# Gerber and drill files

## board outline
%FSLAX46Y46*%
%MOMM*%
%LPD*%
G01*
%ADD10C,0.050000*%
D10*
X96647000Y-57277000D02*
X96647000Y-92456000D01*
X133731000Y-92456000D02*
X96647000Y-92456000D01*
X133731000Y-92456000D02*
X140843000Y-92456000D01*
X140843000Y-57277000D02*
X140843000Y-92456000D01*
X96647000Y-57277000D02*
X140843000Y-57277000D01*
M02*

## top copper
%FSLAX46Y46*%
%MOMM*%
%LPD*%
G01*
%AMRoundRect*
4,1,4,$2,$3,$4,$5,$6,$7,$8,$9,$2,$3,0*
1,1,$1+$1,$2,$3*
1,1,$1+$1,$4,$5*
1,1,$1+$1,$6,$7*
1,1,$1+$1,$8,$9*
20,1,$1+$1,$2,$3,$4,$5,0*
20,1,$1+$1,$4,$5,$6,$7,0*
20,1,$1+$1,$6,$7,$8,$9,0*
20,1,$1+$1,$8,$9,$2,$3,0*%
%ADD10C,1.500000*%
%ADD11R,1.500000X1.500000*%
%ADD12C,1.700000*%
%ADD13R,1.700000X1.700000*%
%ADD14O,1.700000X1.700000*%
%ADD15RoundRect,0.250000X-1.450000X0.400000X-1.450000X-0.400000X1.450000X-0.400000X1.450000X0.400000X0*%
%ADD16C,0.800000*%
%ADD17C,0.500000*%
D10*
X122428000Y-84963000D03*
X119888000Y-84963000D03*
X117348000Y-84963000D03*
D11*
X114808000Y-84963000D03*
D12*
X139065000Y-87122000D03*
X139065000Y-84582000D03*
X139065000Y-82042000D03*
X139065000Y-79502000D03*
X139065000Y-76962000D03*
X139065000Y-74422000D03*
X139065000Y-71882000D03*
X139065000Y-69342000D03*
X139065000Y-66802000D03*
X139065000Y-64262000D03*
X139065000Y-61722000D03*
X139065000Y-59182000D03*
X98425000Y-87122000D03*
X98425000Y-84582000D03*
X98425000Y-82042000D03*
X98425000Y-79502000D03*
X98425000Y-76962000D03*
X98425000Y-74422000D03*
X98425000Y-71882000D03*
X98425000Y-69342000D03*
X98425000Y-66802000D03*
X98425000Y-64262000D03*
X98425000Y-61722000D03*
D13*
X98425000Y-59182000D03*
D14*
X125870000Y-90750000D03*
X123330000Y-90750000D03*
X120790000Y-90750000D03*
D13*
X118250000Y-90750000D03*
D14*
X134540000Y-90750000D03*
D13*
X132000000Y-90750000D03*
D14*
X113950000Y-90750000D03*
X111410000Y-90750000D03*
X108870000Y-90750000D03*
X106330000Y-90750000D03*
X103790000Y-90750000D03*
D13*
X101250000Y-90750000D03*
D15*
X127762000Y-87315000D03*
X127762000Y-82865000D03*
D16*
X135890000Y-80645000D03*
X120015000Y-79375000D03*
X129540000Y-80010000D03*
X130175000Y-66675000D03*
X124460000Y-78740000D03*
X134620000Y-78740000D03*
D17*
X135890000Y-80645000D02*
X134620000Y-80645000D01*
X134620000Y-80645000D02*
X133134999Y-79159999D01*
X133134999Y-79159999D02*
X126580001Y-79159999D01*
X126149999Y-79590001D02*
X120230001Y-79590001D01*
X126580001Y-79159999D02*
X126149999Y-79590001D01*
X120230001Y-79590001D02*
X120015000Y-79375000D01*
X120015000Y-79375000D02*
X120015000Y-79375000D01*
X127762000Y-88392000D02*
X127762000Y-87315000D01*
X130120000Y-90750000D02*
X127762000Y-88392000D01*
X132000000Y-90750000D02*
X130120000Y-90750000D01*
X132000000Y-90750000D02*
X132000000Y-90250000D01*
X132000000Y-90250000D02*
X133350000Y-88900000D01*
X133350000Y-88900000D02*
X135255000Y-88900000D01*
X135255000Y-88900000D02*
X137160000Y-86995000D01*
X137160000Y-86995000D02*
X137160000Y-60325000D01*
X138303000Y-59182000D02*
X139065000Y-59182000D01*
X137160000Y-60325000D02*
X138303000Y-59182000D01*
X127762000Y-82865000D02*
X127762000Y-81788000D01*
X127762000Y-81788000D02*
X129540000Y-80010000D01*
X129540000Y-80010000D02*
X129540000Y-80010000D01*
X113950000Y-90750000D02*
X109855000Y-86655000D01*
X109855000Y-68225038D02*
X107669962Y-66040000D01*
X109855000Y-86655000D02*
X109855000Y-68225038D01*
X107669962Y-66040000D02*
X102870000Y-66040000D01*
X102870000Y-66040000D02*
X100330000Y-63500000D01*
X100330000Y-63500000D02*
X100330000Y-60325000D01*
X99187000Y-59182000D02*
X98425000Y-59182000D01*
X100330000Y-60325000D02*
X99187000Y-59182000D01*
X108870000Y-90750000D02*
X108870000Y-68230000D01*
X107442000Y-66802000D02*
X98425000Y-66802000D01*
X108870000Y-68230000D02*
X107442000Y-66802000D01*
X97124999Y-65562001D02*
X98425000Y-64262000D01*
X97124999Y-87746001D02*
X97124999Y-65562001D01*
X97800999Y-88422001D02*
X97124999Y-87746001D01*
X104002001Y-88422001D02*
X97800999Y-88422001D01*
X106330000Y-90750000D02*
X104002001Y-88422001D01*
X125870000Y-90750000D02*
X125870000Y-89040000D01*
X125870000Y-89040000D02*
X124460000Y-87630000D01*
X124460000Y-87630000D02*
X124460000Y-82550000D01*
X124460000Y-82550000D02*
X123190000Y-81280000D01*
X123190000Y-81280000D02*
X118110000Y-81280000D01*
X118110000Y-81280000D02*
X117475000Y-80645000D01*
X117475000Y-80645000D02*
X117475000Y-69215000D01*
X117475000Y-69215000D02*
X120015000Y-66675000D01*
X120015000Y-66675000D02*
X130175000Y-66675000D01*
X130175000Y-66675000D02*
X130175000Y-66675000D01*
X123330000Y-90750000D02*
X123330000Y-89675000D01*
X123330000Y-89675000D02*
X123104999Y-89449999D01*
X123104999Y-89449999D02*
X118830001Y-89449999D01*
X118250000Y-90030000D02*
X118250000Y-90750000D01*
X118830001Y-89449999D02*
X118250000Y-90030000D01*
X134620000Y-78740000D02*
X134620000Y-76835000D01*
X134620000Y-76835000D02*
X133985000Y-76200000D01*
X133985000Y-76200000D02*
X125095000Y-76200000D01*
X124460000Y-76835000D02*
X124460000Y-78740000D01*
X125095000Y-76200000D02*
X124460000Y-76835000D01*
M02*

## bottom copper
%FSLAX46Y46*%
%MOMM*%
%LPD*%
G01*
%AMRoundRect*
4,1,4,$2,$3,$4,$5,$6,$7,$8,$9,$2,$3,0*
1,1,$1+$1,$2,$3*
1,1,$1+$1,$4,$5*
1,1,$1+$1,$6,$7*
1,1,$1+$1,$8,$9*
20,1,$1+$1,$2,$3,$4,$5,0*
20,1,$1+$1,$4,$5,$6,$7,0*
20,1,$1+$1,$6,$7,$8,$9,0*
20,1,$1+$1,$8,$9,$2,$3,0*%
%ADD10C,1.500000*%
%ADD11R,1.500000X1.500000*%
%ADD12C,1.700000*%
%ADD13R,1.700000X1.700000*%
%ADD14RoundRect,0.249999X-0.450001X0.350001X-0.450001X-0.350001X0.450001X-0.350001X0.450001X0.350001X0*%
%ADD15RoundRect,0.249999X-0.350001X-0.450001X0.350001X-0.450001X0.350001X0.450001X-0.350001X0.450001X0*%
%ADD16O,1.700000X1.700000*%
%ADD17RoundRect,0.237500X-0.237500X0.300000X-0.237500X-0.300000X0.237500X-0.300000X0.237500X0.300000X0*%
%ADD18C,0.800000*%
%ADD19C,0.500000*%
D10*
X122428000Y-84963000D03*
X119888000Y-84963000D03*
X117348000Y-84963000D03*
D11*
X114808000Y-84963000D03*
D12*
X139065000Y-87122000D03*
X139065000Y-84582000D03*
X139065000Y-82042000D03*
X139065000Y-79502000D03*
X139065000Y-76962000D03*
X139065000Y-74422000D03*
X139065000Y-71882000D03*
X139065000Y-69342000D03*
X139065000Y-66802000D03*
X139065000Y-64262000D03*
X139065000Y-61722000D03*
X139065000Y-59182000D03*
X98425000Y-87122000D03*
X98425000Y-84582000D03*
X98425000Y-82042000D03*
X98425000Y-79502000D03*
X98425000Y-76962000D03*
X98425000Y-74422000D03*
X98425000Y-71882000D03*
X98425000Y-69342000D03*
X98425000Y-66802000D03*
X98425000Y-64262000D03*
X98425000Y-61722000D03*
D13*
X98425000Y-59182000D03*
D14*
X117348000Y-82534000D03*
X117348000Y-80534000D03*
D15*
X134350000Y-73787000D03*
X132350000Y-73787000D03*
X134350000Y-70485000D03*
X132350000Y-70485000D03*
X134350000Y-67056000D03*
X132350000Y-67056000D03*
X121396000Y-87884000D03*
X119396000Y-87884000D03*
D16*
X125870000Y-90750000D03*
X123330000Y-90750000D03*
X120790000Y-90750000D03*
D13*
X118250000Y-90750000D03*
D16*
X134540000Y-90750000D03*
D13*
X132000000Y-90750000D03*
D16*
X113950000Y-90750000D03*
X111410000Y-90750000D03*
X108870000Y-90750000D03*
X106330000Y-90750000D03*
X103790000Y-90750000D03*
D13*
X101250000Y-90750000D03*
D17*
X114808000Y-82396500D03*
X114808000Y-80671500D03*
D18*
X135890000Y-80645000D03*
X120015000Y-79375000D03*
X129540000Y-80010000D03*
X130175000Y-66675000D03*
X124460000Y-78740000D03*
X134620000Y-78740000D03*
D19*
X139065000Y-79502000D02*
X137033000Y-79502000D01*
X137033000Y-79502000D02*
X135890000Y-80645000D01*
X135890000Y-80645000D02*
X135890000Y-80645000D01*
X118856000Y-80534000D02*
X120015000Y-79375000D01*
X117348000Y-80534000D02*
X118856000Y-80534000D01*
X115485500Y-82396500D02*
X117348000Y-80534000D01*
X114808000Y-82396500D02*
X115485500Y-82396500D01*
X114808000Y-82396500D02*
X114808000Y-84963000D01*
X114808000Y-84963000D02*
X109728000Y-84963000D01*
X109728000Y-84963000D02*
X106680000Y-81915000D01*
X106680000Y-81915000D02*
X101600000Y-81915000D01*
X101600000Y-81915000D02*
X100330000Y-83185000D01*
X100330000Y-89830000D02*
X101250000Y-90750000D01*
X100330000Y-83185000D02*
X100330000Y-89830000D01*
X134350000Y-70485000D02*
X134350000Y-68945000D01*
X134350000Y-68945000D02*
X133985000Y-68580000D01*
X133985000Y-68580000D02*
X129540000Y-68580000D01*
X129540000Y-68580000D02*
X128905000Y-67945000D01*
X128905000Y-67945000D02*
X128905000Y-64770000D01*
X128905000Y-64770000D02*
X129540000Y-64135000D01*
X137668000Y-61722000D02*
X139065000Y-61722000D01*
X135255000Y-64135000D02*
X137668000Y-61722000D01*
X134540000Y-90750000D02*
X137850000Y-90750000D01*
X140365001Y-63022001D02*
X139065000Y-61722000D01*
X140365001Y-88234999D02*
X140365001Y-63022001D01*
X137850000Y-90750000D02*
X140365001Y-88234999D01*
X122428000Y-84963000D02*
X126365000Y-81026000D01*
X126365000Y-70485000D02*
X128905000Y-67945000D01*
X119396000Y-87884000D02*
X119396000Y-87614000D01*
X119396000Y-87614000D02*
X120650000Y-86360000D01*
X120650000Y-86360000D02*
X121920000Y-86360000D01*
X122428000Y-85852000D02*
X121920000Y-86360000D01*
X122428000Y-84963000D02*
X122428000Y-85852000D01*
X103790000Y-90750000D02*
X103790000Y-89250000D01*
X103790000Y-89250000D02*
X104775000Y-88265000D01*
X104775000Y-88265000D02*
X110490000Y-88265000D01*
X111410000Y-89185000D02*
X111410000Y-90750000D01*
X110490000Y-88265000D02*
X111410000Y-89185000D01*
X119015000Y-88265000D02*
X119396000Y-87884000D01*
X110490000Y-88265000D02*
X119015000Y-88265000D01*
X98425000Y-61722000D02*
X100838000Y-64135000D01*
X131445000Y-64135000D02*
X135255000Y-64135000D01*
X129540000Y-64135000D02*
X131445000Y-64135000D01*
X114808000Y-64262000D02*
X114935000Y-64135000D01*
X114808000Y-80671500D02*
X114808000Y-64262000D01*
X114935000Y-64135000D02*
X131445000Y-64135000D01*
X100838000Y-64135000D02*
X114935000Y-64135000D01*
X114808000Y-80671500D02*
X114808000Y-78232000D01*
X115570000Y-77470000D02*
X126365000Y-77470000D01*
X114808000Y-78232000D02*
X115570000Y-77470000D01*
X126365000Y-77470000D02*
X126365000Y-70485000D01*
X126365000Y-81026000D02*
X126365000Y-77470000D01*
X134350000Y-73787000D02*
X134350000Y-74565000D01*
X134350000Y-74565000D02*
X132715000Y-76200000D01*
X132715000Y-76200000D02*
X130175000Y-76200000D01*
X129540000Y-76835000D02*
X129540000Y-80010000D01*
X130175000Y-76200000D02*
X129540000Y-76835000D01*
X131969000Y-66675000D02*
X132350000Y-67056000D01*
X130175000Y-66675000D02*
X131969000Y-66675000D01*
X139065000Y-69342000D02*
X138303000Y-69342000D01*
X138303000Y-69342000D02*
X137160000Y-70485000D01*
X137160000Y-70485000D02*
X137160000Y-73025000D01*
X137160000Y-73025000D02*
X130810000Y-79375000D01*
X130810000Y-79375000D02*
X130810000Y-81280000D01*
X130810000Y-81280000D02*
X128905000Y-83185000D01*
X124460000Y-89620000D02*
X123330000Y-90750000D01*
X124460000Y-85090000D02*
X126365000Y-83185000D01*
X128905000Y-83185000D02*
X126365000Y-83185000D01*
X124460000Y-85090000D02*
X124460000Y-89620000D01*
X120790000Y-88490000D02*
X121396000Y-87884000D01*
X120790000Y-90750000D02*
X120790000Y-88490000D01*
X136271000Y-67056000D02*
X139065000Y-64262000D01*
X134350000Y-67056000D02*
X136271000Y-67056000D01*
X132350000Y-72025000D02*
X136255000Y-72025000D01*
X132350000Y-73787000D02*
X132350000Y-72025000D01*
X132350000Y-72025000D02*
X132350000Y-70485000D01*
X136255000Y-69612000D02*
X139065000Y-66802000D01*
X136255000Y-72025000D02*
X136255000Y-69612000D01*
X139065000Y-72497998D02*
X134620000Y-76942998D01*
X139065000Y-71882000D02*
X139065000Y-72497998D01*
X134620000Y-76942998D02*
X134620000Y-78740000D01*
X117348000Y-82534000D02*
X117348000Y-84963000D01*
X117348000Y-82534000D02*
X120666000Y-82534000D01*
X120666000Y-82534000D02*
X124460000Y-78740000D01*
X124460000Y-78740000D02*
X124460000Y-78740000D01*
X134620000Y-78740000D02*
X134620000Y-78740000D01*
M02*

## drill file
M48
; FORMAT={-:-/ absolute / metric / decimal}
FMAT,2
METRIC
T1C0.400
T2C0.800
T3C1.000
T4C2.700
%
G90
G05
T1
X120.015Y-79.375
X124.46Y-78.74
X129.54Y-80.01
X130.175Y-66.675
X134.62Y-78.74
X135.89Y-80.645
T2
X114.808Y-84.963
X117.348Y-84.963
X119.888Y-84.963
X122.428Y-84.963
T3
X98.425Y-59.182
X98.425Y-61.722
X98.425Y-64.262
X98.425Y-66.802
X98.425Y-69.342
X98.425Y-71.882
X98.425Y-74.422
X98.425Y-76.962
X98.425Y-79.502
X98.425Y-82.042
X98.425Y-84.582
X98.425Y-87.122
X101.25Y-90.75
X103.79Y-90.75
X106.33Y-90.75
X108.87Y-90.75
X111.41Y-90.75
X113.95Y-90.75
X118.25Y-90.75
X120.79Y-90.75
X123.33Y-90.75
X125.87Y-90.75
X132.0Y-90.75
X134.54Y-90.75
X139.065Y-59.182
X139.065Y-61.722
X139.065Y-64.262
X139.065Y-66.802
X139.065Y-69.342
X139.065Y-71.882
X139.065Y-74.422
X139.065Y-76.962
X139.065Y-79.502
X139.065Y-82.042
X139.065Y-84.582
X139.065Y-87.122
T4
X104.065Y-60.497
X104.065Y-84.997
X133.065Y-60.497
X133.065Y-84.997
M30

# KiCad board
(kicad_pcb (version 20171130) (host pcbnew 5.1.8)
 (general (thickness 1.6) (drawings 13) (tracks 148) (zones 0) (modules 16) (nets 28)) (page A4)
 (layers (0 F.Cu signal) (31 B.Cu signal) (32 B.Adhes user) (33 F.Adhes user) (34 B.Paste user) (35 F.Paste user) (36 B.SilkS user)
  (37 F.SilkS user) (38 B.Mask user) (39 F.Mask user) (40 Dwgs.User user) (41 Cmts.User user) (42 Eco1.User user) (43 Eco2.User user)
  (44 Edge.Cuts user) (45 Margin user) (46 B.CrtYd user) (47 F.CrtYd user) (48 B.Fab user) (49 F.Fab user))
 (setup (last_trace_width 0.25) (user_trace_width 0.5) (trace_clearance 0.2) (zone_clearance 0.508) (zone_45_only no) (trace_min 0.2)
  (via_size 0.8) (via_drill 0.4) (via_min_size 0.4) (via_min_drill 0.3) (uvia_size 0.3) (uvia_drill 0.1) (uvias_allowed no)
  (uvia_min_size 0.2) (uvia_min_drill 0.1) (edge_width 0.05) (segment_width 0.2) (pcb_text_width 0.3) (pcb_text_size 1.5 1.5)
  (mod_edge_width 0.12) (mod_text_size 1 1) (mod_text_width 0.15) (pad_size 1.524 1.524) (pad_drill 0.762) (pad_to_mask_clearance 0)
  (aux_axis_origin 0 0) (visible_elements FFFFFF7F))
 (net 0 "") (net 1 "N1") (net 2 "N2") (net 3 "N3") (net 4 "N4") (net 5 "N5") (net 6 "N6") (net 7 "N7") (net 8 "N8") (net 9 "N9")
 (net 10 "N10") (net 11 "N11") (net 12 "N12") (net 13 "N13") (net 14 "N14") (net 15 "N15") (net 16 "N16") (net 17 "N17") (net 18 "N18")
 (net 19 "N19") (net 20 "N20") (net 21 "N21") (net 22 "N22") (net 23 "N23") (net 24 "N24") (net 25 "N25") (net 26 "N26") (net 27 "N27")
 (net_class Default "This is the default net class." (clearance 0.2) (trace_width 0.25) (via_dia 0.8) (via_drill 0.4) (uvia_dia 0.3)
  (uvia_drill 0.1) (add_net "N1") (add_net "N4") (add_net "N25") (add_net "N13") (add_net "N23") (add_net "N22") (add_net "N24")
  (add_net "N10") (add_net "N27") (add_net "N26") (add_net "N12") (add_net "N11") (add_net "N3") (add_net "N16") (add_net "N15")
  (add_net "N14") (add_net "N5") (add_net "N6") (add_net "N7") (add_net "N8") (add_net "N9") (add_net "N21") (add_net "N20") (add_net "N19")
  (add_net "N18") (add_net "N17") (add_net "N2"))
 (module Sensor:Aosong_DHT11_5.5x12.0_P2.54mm (layer F.Cu) (at 114.808 84.963 90)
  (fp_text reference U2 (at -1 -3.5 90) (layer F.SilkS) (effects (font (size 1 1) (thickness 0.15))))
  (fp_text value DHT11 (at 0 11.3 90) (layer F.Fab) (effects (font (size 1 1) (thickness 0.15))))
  (pad 4 thru_hole circle (at 0 7.62 90) (size 1.5 1.5) (drill 0.8) (layers *.Cu *.Mask) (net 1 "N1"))
  (pad 3 thru_hole circle (at 0 5.08 90) (size 1.5 1.5) (drill 0.8) (layers *.Cu *.Mask) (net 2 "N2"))
  (pad 2 thru_hole circle (at 0 2.54 90) (size 1.5 1.5) (drill 0.8) (layers *.Cu *.Mask) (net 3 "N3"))
  (pad 1 thru_hole rect (at 0 0 90) (size 1.5 1.5) (drill 0.8) (layers *.Cu *.Mask) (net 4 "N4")))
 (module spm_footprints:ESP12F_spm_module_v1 (layer F.Cu) (at 118.745 57.277)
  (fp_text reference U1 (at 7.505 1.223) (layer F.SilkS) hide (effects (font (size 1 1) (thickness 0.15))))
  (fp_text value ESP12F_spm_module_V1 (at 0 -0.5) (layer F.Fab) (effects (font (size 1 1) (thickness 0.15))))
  (pad 13 thru_hole circle (at 20.32 29.845) (size 1.7 1.7) (drill 1) (layers *.Cu *.Mask) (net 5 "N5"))
  (pad 14 thru_hole circle (at 20.32 27.305) (size 1.7 1.7) (drill 1) (layers *.Cu *.Mask) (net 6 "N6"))
  (pad 15 thru_hole circle (at 20.32 24.765) (size 1.7 1.7) (drill 1) (layers *.Cu *.Mask) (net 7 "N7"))
  (pad 16 thru_hole circle (at 20.32 22.225) (size 1.7 1.7) (drill 1) (layers *.Cu *.Mask) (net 4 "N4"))
  (pad 17 thru_hole circle (at 20.32 19.685) (size 1.7 1.7) (drill 1) (layers *.Cu *.Mask) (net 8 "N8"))
  (pad 18 thru_hole circle (at 20.32 17.145) (size 1.7 1.7) (drill 1) (layers *.Cu *.Mask) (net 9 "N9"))
  (pad 19 thru_hole circle (at 20.32 14.605) (size 1.7 1.7) (drill 1) (layers *.Cu *.Mask) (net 3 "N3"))
  (pad 20 thru_hole circle (at 20.32 12.065) (size 1.7 1.7) (drill 1) (layers *.Cu *.Mask) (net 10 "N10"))
  (pad 21 thru_hole circle (at 20.32 9.525) (size 1.7 1.7) (drill 1) (layers *.Cu *.Mask) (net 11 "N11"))
  (pad 22 thru_hole circle (at 20.32 6.985) (size 1.7 1.7) (drill 1) (layers *.Cu *.Mask) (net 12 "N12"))
  (pad 23 thru_hole circle (at 20.32 4.445) (size 1.7 1.7) (drill 1) (layers *.Cu *.Mask) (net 1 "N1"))
  (pad 24 thru_hole circle (at 20.32 1.905) (size 1.7 1.7) (drill 1) (layers *.Cu *.Mask) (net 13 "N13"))
  (pad 12 thru_hole circle (at -20.32 29.845) (size 1.7 1.7) (drill 1) (layers *.Cu *.Mask) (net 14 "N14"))
  (pad 11 thru_hole circle (at -20.32 27.305) (size 1.7 1.7) (drill 1) (layers *.Cu *.Mask) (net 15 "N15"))
  (pad 10 thru_hole circle (at -20.32 24.765) (size 1.7 1.7) (drill 1) (layers *.Cu *.Mask) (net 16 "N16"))
  (pad 9 thru_hole circle (at -20.32 22.225) (size 1.7 1.7) (drill 1) (layers *.Cu *.Mask) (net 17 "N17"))
  (pad 8 thru_hole circle (at -20.32 19.685) (size 1.7 1.7) (drill 1) (layers *.Cu *.Mask) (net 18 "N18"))
  (pad 7 thru_hole circle (at -20.32 17.145) (size 1.7 1.7) (drill 1) (layers *.Cu *.Mask) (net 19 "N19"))
  (pad 6 thru_hole circle (at -20.32 14.605) (size 1.7 1.7) (drill 1) (layers *.Cu *.Mask) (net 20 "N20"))
  (pad 5 thru_hole circle (at -20.32 12.065) (size 1.7 1.7) (drill 1) (layers *.Cu *.Mask) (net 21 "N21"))
  (pad 4 thru_hole circle (at -20.32 9.525) (size 1.7 1.7) (drill 1) (layers *.Cu *.Mask) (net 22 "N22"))
  (pad 3 thru_hole circle (at -20.32 6.985) (size 1.7 1.7) (drill 1) (layers *.Cu *.Mask) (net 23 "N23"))
  (pad 2 thru_hole circle (at -20.32 4.445) (size 1.7 1.7) (drill 1) (layers *.Cu *.Mask) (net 1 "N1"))
  (pad 1 thru_hole rect (at -20.32 1.905) (size 1.7 1.7) (drill 1) (layers *.Cu *.Mask) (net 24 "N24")))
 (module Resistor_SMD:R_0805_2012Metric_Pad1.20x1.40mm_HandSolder (layer B.Cu) (at 117.348 81.534 270)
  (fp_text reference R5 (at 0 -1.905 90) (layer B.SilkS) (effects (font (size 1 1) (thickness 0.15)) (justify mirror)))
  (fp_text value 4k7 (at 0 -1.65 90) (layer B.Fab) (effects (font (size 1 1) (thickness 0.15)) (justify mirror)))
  (pad 2 smd roundrect (at 1 0 270) (size 1.2 1.4) (layers B.Cu B.Paste B.Mask) (roundrect_rratio 0.2083325) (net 3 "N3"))
  (pad 1 smd roundrect (at -1 0 270) (size 1.2 1.4) (layers B.Cu B.Paste B.Mask) (roundrect_rratio 0.2083325) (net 4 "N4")))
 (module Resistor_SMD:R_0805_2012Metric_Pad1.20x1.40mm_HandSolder (layer B.Cu) (at 133.35 73.787)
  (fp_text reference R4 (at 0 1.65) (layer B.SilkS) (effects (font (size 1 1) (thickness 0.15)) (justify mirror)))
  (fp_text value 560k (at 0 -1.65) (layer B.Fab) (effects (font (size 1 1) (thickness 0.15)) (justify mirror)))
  (pad 2 smd roundrect (at 1 0) (size 1.2 1.4) (layers B.Cu B.Paste B.Mask) (roundrect_rratio 0.2083325) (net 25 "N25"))
  (pad 1 smd roundrect (at -1 0) (size 1.2 1.4) (layers B.Cu B.Paste B.Mask) (roundrect_rratio 0.2083325) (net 11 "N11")))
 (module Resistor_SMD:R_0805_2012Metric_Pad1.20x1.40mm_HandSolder (layer B.Cu) (at 133.35 70.485)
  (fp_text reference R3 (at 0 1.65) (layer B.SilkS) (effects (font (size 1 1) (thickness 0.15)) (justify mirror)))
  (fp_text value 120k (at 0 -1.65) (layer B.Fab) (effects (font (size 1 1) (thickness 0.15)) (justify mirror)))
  (pad 2 smd roundrect (at 1 0) (size 1.2 1.4) (layers B.Cu B.Paste B.Mask) (roundrect_rratio 0.2083325) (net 1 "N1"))
  (pad 1 smd roundrect (at -1 0) (size 1.2 1.4) (layers B.Cu B.Paste B.Mask) (roundrect_rratio 0.2083325) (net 11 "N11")))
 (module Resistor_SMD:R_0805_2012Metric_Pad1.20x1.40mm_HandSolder (layer B.Cu) (at 133.35 67.056)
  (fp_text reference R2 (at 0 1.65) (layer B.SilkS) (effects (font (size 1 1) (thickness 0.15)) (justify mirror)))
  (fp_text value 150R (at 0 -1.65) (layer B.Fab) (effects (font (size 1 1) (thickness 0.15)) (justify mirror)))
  (pad 2 smd roundrect (at 1 0) (size 1.2 1.4) (layers B.Cu B.Paste B.Mask) (roundrect_rratio 0.2083325) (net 12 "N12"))
  (pad 1 smd roundrect (at -1 0) (size 1.2 1.4) (layers B.Cu B.Paste B.Mask) (roundrect_rratio 0.2083325) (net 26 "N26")))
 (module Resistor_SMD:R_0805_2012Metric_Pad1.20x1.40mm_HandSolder (layer B.Cu) (at 120.396 87.884)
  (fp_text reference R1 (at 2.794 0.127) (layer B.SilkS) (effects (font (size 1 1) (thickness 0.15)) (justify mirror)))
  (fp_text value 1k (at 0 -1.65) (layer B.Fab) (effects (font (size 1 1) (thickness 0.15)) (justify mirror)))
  (pad 2 smd roundrect (at 1 0) (size 1.2 1.4) (layers B.Cu B.Paste B.Mask) (roundrect_rratio 0.2083325) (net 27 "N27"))
  (pad 1 smd roundrect (at -1 0) (size 1.2 1.4) (layers B.Cu B.Paste B.Mask) (roundrect_rratio 0.2083325) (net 1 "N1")))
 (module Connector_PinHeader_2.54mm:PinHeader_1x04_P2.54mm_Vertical (layer F.Cu) (at 118.25 90.75 90)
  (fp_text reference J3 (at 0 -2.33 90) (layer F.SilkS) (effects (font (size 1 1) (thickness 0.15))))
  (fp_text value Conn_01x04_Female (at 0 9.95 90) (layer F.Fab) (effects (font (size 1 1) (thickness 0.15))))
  (pad 4 thru_hole oval (at 0 7.62 90) (size 1.7 1.7) (drill 1) (layers *.Cu *.Mask) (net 26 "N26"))
  (pad 3 thru_hole oval (at 0 5.08 90) (size 1.7 1.7) (drill 1) (layers *.Cu *.Mask) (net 10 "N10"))
  (pad 2 thru_hole oval (at 0 2.54 90) (size 1.7 1.7) (drill 1) (layers *.Cu *.Mask) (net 27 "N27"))
  (pad 1 thru_hole rect (at 0 0 90) (size 1.7 1.7) (drill 1) (layers *.Cu *.Mask) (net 10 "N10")))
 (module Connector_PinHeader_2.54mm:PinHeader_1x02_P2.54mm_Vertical (layer F.Cu) (at 132 90.75 90)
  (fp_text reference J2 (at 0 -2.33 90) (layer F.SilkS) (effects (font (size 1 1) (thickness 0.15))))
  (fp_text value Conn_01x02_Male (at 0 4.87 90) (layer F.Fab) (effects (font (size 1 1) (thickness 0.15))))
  (pad 2 thru_hole oval (at 0 2.54 90) (size 1.7 1.7) (drill 1) (layers *.Cu *.Mask) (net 1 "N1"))
  (pad 1 thru_hole rect (at 0 0 90) (size 1.7 1.7) (drill 1) (layers *.Cu *.Mask) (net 13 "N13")))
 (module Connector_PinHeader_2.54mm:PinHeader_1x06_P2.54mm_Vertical (layer F.Cu) (at 101.25 90.75 90)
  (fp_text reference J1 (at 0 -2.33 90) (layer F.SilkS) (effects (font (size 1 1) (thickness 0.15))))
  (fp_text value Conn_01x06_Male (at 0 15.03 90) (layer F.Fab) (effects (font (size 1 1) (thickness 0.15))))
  (pad 6 thru_hole oval (at 0 12.7 90) (size 1.7 1.7) (drill 1) (layers *.Cu *.Mask) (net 24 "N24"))
  (pad 5 thru_hole oval (at 0 10.16 90) (size 1.7 1.7) (drill 1) (layers *.Cu *.Mask) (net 1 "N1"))
  (pad 4 thru_hole oval (at 0 7.62 90) (size 1.7 1.7) (drill 1) (layers *.Cu *.Mask) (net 22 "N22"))
  (pad 3 thru_hole oval (at 0 5.08 90) (size 1.7 1.7) (drill 1) (layers *.Cu *.Mask) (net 23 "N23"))
  (pad 2 thru_hole oval (at 0 2.54 90) (size 1.7 1.7) (drill 1) (layers *.Cu *.Mask) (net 1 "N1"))
  (pad 1 thru_hole rect (at 0 0 90) (size 1.7 1.7) (drill 1) (layers *.Cu *.Mask) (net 4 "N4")))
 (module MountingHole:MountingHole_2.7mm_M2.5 (layer F.Cu) (at 133.065 84.997)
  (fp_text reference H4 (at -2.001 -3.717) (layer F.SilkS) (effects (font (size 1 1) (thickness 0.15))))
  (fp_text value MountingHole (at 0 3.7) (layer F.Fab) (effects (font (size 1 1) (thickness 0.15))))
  (pad 1 np_thru_hole circle (at 0 0) (size 2.7 2.7) (drill 2.7) (layers *.Cu *.Mask)))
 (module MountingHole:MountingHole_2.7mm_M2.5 (layer F.Cu) (at 133.065 60.497)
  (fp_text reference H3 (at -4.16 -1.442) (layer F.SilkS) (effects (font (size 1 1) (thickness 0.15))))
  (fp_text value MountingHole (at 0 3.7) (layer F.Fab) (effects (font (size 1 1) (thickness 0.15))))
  (pad 1 np_thru_hole circle (at 0 0) (size 2.7 2.7) (drill 2.7) (layers *.Cu *.Mask)))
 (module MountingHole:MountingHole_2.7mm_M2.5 (layer F.Cu) (at 104.065 84.997)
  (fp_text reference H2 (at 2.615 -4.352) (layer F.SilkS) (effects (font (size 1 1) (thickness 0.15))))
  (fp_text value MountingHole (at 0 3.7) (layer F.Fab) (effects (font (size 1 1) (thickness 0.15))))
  (pad 1 np_thru_hole circle (at 0 0) (size 2.7 2.7) (drill 2.7) (layers *.Cu *.Mask)))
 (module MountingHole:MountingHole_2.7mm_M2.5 (layer F.Cu) (at 104.065 60.497)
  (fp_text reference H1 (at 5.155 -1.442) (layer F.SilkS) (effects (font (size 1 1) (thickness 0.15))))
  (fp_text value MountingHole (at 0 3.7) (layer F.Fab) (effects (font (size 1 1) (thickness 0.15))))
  (pad 1 np_thru_hole circle (at 0 0) (size 2.7 2.7) (drill 2.7) (layers *.Cu *.Mask)))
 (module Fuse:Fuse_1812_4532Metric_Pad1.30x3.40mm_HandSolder (layer F.Cu) (at 127.762 85.09 270)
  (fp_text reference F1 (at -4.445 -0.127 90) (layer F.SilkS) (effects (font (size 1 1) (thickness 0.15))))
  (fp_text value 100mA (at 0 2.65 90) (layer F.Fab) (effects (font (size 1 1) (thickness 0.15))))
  (pad 2 smd roundrect (at 2.225 0 270) (size 1.3 3.4) (layers F.Cu F.Paste F.Mask) (roundrect_rratio 0.1923076923076923) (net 13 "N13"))
  (pad 1 smd roundrect (at -2.225 0 270) (size 1.3 3.4) (layers F.Cu F.Paste F.Mask) (roundrect_rratio 0.1923076923076923) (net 25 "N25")))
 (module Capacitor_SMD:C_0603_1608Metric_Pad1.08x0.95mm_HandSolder (layer B.Cu) (at 114.808 81.534 270)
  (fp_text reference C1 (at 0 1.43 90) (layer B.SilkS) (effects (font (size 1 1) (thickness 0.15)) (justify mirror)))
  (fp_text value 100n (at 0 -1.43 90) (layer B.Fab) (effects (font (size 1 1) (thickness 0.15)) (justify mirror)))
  (pad 2 smd roundrect (at 0.8625 0 270) (size 1.075 0.95) (layers B.Cu B.Paste B.Mask) (roundrect_rratio 0.25) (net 4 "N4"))
  (pad 1 smd roundrect (at -0.8625 0 270) (size 1.075 0.95) (layers B.Cu B.Paste B.Mask) (roundrect_rratio 0.25) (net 1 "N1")))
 (gr_line (start 96.647 57.277) (end 96.647 92.456) (layer Edge.Cuts) (width 0.05))
 (gr_line (start 133.731 92.456) (end 96.647 92.456) (layer Edge.Cuts) (width 0.05))
 (gr_line (start 133.731 92.456) (end 140.843 92.456) (layer Edge.Cuts) (width 0.05))
 (gr_line (start 140.843 57.277) (end 140.843 92.456) (layer Edge.Cuts) (width 0.05))
 (gr_line (start 96.647 57.277) (end 140.843 57.277) (layer Edge.Cuts) (width 0.05))
 (segment (start 139.065 79.502) (end 137.033 79.502) (width 0.5) (layer B.Cu) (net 4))
 (segment (start 137.033 79.502) (end 135.89 80.645) (width 0.5) (layer B.Cu) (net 4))
 (segment (start 135.89 80.645) (end 135.89 80.645) (width 0.5) (layer B.Cu) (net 4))
 (via (at 135.89 80.645) (size 0.8) (drill 0.4) (layers F.Cu B.Cu) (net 4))
 (segment (start 135.89 80.645) (end 134.62 80.645) (width 0.5) (layer F.Cu) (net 4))
 (segment (start 134.62 80.645) (end 133.134999 79.159999) (width 0.5) (layer F.Cu) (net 4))
 (segment (start 133.134999 79.159999) (end 126.580001 79.159999) (width 0.5) (layer F.Cu) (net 4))
 (segment (start 126.149999 79.590001) (end 120.230001 79.590001) (width 0.5) (layer F.Cu) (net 4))
 (segment (start 126.580001 79.159999) (end 126.149999 79.590001) (width 0.5) (layer F.Cu) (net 4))
 (segment (start 120.230001 79.590001) (end 120.015 79.375) (width 0.5) (layer F.Cu) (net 4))
 (segment (start 120.015 79.375) (end 120.015 79.375) (width 0.5) (layer F.Cu) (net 4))
 (via (at 120.015 79.375) (size 0.8) (drill 0.4) (layers F.Cu B.Cu) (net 4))
 (segment (start 118.856 80.534) (end 120.015 79.375) (width 0.5) (layer B.Cu) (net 4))
 (segment (start 117.348 80.534) (end 118.856 80.534) (width 0.5) (layer B.Cu) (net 4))
 (segment (start 115.4855 82.3965) (end 117.348 80.534) (width 0.5) (layer B.Cu) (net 4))
 (segment (start 114.808 82.3965) (end 115.4855 82.3965) (width 0.5) (layer B.Cu) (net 4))
 (segment (start 114.808 82.3965) (end 114.808 84.963) (width 0.5) (layer B.Cu) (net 4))
 (segment (start 114.808 84.963) (end 109.728 84.963) (width 0.5) (layer B.Cu) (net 4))
 (segment (start 109.728 84.963) (end 106.68 81.915) (width 0.5) (layer B.Cu) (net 4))
 (segment (start 106.68 81.915) (end 101.6 81.915) (width 0.5) (layer B.Cu) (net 4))
 (segment (start 101.6 81.915) (end 100.33 83.185) (width 0.5) (layer B.Cu) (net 4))
 (segment (start 100.33 89.83) (end 101.25 90.75) (width 0.5) (layer B.Cu) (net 4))
 (segment (start 100.33 83.185) (end 100.33 89.83) (width 0.5) (layer B.Cu) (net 4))
 (segment (start 134.35 70.485) (end 134.35 68.945) (width 0.5) (layer B.Cu) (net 1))
 (segment (start 134.35 68.945) (end 133.985 68.58) (width 0.5) (layer B.Cu) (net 1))
 (segment (start 133.985 68.58) (end 129.54 68.58) (width 0.5) (layer B.Cu) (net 1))
 (segment (start 129.54 68.58) (end 128.905 67.945) (width 0.5) (layer B.Cu) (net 1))
 (segment (start 128.905 67.945) (end 128.905 64.77) (width 0.5) (layer B.Cu) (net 1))
 (segment (start 128.905 64.77) (end 129.54 64.135) (width 0.5) (layer B.Cu) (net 1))
 (segment (start 137.668 61.722) (end 139.065 61.722) (width 0.5) (layer B.Cu) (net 1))
 (segment (start 135.255 64.135) (end 137.668 61.722) (width 0.5) (layer B.Cu) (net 1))
 (segment (start 134.54 90.75) (end 137.85 90.75) (width 0.5) (layer B.Cu) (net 1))
 (segment (start 140.365001 63.022001) (end 139.065 61.722) (width 0.5) (layer B.Cu) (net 1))
 (segment (start 140.365001 88.234999) (end 140.365001 63.022001) (width 0.5) (layer B.Cu) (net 1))
 (segment (start 137.85 90.75) (end 140.365001 88.234999) (width 0.5) (layer B.Cu) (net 1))
 (segment (start 122.428 84.963) (end 126.365 81.026) (width 0.5) (layer B.Cu) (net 1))
 (segment (start 126.365 70.485) (end 128.905 67.945) (width 0.5) (layer B.Cu) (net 1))
 (segment (start 119.396 87.884) (end 119.396 87.614) (width 0.5) (layer B.Cu) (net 1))
 (segment (start 119.396 87.614) (end 120.65 86.36) (width 0.5) (layer B.Cu) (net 1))
 (segment (start 120.65 86.36) (end 121.92 86.36) (width 0.5) (layer B.Cu) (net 1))
 (segment (start 122.428 85.852) (end 121.92 86.36) (width 0.5) (layer B.Cu) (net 1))
 (segment (start 122.428 84.963) (end 122.428 85.852) (width 0.5) (layer B.Cu) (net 1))
 (segment (start 103.79 90.75) (end 103.79 89.25) (width 0.5) (layer B.Cu) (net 1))
 (segment (start 103.79 89.25) (end 104.775 88.265) (width 0.5) (layer B.Cu) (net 1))
 (segment (start 104.775 88.265) (end 110.49 88.265) (width 0.5) (layer B.Cu) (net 1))
 (segment (start 111.41 89.185) (end 111.41 90.75) (width 0.5) (layer B.Cu) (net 1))
 (segment (start 110.49 88.265) (end 111.41 89.185) (width 0.5) (layer B.Cu) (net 1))
 (segment (start 119.015 88.265) (end 119.396 87.884) (width 0.5) (layer B.Cu) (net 1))
 (segment (start 110.49 88.265) (end 119.015 88.265) (width 0.5) (layer B.Cu) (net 1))
 (segment (start 98.425 61.722) (end 100.838 64.135) (width 0.5) (layer B.Cu) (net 1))
 (segment (start 131.445 64.135) (end 135.255 64.135) (width 0.5) (layer B.Cu) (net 1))
 (segment (start 129.54 64.135) (end 131.445 64.135) (width 0.5) (layer B.Cu) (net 1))
 (segment (start 114.808 64.262) (end 114.935 64.135) (width 0.5) (layer B.Cu) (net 1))
 (segment (start 114.808 80.6715) (end 114.808 64.262) (width 0.5) (layer B.Cu) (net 1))
 (segment (start 114.935 64.135) (end 131.445 64.135) (width 0.5) (layer B.Cu) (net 1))
 (segment (start 100.838 64.135) (end 114.935 64.135) (width 0.5) (layer B.Cu) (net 1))
 (segment (start 114.808 80.6715) (end 114.808 78.232) (width 0.5) (layer B.Cu) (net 1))
 (segment (start 115.57 77.47) (end 126.365 77.47) (width 0.5) (layer B.Cu) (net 1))
 (segment (start 114.808 78.232) (end 115.57 77.47) (width 0.5) (layer B.Cu) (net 1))
 (segment (start 126.365 77.47) (end 126.365 70.485) (width 0.5) (layer B.Cu) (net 1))
 (segment (start 126.365 81.026) (end 126.365 77.47) (width 0.5) (layer B.Cu) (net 1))
 (segment (start 127.762 88.392) (end 127.762 87.315) (width 0.5) (layer F.Cu) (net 13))
 (segment (start 130.12 90.75) (end 127.762 88.392) (width 0.5) (layer F.Cu) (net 13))
 (segment (start 132 90.75) (end 130.12 90.75) (width 0.5) (layer F.Cu) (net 13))
 (segment (start 132 90.75) (end 132 90.25) (width 0.5) (layer F.Cu) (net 13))
 (segment (start 132 90.25) (end 133.35 88.9) (width 0.5) (layer F.Cu) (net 13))
 (segment (start 133.35 88.9) (end 135.255 88.9) (width 0.5) (layer F.Cu) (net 13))
 (segment (start 135.255 88.9) (end 137.16 86.995) (width 0.5) (layer F.Cu) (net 13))
 (segment (start 137.16 86.995) (end 137.16 60.325) (width 0.5) (layer F.Cu) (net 13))
 (segment (start 138.303 59.182) (end 139.065 59.182) (width 0.5) (layer F.Cu) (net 13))
 (segment (start 137.16 60.325) (end 138.303 59.182) (width 0.5) (layer F.Cu) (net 13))
 (segment (start 127.762 82.865) (end 127.762 81.788) (width 0.5) (layer F.Cu) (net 25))
 (segment (start 127.762 81.788) (end 129.54 80.01) (width 0.5) (layer F.Cu) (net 25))
 (segment (start 129.54 80.01) (end 129.54 80.01) (width 0.5) (layer F.Cu) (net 25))
 (via (at 129.54 80.01) (size 0.8) (drill 0.4) (layers F.Cu B.Cu) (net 25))
 (segment (start 134.35 73.787) (end 134.35 74.565) (width 0.5) (layer B.Cu) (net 25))
 (segment (start 134.35 74.565) (end 132.715 76.2) (width 0.5) (layer B.Cu) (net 25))
 (segment (start 132.715 76.2) (end 130.175 76.2) (width 0.5) (layer B.Cu) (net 25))
 (segment (start 129.54 76.835) (end 129.54 80.01) (width 0.5) (layer B.Cu) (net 25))
 (segment (start 130.175 76.2) (end 129.54 76.835) (width 0.5) (layer B.Cu) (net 25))
 (segment (start 113.95 90.75) (end 109.855 86.655) (width 0.5) (layer F.Cu) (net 24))
 (segment (start 109.855 68.225038) (end 107.669962 66.04) (width 0.5) (layer F.Cu) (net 24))
 (segment (start 109.855 86.655) (end 109.855 68.225038) (width 0.5) (layer F.Cu) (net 24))
 (segment (start 107.669962 66.04) (end 102.87 66.04) (width 0.5) (layer F.Cu) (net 24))
 (segment (start 102.87 66.04) (end 100.33 63.5) (width 0.5) (layer F.Cu) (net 24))
 (segment (start 100.33 63.5) (end 100.33 60.325) (width 0.5) (layer F.Cu) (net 24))
 (segment (start 99.187 59.182) (end 98.425 59.182) (width 0.5) (layer F.Cu) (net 24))
 (segment (start 100.33 60.325) (end 99.187 59.182) (width 0.5) (layer F.Cu) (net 24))
 (segment (start 108.87 90.75) (end 108.87 68.23) (width 0.5) (layer F.Cu) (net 22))
 (segment (start 107.442 66.802) (end 98.425 66.802) (width 0.5) (layer F.Cu) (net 22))
 (segment (start 108.87 68.23) (end 107.442 66.802) (width 0.5) (layer F.Cu) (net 22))
 (segment (start 97.124999 65.562001) (end 98.425 64.262) (width 0.5) (layer F.Cu) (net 23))
 (segment (start 97.124999 87.746001) (end 97.124999 65.562001) (width 0.5) (layer F.Cu) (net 23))
 (segment (start 97.800999 88.422001) (end 97.124999 87.746001) (width 0.5) (layer F.Cu) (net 23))
 (segment (start 104.002001 88.422001) (end 97.800999 88.422001) (width 0.5) (layer F.Cu) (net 23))
 (segment (start 106.33 90.75) (end 104.002001 88.422001) (width 0.5) (layer F.Cu) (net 23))
 (segment (start 125.87 90.75) (end 125.87 89.04) (width 0.5) (layer F.Cu) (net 26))
 (segment (start 125.87 89.04) (end 124.46 87.63) (width 0.5) (layer F.Cu) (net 26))
 (segment (start 124.46 87.63) (end 124.46 82.55) (width 0.5) (layer F.Cu) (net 26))
 (segment (start 124.46 82.55) (end 123.19 81.28) (width 0.5) (layer F.Cu) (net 26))
 (segment (start 123.19 81.28) (end 118.11 81.28) (width 0.5) (layer F.Cu) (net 26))
 (segment (start 118.11 81.28) (end 117.475 80.645) (width 0.5) (layer F.Cu) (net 26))
 (segment (start 117.475 80.645) (end 117.475 69.215) (width 0.5) (layer F.Cu) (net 26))
 (segment (start 117.475 69.215) (end 120.015 66.675) (width 0.5) (layer F.Cu) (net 26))
 (segment (start 120.015 66.675) (end 130.175 66.675) (width 0.5) (layer F.Cu) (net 26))
 (segment (start 130.175 66.675) (end 130.175 66.675) (width 0.5) (layer F.Cu) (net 26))
 (via (at 130.175 66.675) (size 0.8) (drill 0.4) (layers F.Cu B.Cu) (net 26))
 (segment (start 131.969 66.675) (end 132.35 67.056) (width 0.5) (layer B.Cu) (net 26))
 (segment (start 130.175 66.675) (end 131.969 66.675) (width 0.5) (layer B.Cu) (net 26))
 (segment (start 139.065 69.342) (end 138.303 69.342) (width 0.5) (layer B.Cu) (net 10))
 (segment (start 138.303 69.342) (end 137.16 70.485) (width 0.5) (layer B.Cu) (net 10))
 (segment (start 137.16 70.485) (end 137.16 73.025) (width 0.5) (layer B.Cu) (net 10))
 (segment (start 137.16 73.025) (end 130.81 79.375) (width 0.5) (layer B.Cu) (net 10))
 (segment (start 130.81 79.375) (end 130.81 81.28) (width 0.5) (layer B.Cu) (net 10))
 (segment (start 130.81 81.28) (end 128.905 83.185) (width 0.5) (layer B.Cu) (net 10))
 (segment (start 124.46 89.62) (end 123.33 90.75) (width 0.5) (layer B.Cu) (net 10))
 (segment (start 124.46 85.09) (end 126.365 83.185) (width 0.5) (layer B.Cu) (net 10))
 (segment (start 128.905 83.185) (end 126.365 83.185) (width 0.5) (layer B.Cu) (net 10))
 (segment (start 124.46 85.09) (end 124.46 89.62) (width 0.5) (layer B.Cu) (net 10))
 (segment (start 123.33 90.75) (end 123.33 89.675) (width 0.5) (layer F.Cu) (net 10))
 (segment (start 123.33 89.675) (end 123.104999 89.449999) (width 0.5) (layer F.Cu) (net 10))
 (segment (start 123.104999 89.449999) (end 118.830001 89.449999) (width 0.5) (layer F.Cu) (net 10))
 (segment (start 118.25 90.03) (end 118.25 90.75) (width 0.5) (layer F.Cu) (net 10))
 (segment (start 118.830001 89.449999) (end 118.25 90.03) (width 0.5) (layer F.Cu) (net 10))
 (segment (start 120.79 88.49) (end 121.396 87.884) (width 0.5) (layer B.Cu) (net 27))
 (segment (start 120.79 90.75) (end 120.79 88.49) (width 0.5) (layer B.Cu) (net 27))
 (segment (start 136.271 67.056) (end 139.065 64.262) (width 0.5) (layer B.Cu) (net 12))
 (segment (start 134.35 67.056) (end 136.271 67.056) (width 0.5) (layer B.Cu) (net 12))
 (segment (start 132.35 72.025) (end 136.255 72.025) (width 0.5) (layer B.Cu) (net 11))
 (segment (start 132.35 73.787) (end 132.35 72.025) (width 0.5) (layer B.Cu) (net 11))
 (segment (start 132.35 72.025) (end 132.35 70.485) (width 0.5) (layer B.Cu) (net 11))
 (segment (start 136.255 69.612) (end 139.065 66.802) (width 0.5) (layer B.Cu) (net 11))
 (segment (start 136.255 72.025) (end 136.255 69.612) (width 0.5) (layer B.Cu) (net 11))
 (segment (start 139.065 72.497998) (end 134.62 76.942998) (width 0.5) (layer B.Cu) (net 3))
 (segment (start 139.065 71.882) (end 139.065 72.497998) (width 0.5) (layer B.Cu) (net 3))
 (segment (start 134.62 76.942998) (end 134.62 78.74) (width 0.5) (layer B.Cu) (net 3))
 (segment (start 117.348 82.534) (end 117.348 84.963) (width 0.5) (layer B.Cu) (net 3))
 (segment (start 117.348 82.534) (end 120.666 82.534) (width 0.5) (layer B.Cu) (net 3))
 (segment (start 120.666 82.534) (end 124.46 78.74) (width 0.5) (layer B.Cu) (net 3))
 (segment (start 124.46 78.74) (end 124.46 78.74) (width 0.5) (layer B.Cu) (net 3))
 (via (at 124.46 78.74) (size 0.8) (drill 0.4) (layers F.Cu B.Cu) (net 3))
 (segment (start 134.62 78.74) (end 134.62 78.74) (width 0.5) (layer B.Cu) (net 3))
 (via (at 134.62 78.74) (size 0.8) (drill 0.4) (layers F.Cu B.Cu) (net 3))
 (segment (start 134.62 78.74) (end 134.62 76.835) (width 0.5) (layer F.Cu) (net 3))
 (segment (start 134.62 76.835) (end 133.985 76.2) (width 0.5) (layer F.Cu) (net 3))
 (segment (start 133.985 76.2) (end 125.095 76.2) (width 0.5) (layer F.Cu) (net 3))
 (segment (start 124.46 76.835) (end 124.46 78.74) (width 0.5) (layer F.Cu) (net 3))
 (segment (start 125.095 76.2) (end 124.46 76.835) (width 0.5) (layer F.Cu) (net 3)))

